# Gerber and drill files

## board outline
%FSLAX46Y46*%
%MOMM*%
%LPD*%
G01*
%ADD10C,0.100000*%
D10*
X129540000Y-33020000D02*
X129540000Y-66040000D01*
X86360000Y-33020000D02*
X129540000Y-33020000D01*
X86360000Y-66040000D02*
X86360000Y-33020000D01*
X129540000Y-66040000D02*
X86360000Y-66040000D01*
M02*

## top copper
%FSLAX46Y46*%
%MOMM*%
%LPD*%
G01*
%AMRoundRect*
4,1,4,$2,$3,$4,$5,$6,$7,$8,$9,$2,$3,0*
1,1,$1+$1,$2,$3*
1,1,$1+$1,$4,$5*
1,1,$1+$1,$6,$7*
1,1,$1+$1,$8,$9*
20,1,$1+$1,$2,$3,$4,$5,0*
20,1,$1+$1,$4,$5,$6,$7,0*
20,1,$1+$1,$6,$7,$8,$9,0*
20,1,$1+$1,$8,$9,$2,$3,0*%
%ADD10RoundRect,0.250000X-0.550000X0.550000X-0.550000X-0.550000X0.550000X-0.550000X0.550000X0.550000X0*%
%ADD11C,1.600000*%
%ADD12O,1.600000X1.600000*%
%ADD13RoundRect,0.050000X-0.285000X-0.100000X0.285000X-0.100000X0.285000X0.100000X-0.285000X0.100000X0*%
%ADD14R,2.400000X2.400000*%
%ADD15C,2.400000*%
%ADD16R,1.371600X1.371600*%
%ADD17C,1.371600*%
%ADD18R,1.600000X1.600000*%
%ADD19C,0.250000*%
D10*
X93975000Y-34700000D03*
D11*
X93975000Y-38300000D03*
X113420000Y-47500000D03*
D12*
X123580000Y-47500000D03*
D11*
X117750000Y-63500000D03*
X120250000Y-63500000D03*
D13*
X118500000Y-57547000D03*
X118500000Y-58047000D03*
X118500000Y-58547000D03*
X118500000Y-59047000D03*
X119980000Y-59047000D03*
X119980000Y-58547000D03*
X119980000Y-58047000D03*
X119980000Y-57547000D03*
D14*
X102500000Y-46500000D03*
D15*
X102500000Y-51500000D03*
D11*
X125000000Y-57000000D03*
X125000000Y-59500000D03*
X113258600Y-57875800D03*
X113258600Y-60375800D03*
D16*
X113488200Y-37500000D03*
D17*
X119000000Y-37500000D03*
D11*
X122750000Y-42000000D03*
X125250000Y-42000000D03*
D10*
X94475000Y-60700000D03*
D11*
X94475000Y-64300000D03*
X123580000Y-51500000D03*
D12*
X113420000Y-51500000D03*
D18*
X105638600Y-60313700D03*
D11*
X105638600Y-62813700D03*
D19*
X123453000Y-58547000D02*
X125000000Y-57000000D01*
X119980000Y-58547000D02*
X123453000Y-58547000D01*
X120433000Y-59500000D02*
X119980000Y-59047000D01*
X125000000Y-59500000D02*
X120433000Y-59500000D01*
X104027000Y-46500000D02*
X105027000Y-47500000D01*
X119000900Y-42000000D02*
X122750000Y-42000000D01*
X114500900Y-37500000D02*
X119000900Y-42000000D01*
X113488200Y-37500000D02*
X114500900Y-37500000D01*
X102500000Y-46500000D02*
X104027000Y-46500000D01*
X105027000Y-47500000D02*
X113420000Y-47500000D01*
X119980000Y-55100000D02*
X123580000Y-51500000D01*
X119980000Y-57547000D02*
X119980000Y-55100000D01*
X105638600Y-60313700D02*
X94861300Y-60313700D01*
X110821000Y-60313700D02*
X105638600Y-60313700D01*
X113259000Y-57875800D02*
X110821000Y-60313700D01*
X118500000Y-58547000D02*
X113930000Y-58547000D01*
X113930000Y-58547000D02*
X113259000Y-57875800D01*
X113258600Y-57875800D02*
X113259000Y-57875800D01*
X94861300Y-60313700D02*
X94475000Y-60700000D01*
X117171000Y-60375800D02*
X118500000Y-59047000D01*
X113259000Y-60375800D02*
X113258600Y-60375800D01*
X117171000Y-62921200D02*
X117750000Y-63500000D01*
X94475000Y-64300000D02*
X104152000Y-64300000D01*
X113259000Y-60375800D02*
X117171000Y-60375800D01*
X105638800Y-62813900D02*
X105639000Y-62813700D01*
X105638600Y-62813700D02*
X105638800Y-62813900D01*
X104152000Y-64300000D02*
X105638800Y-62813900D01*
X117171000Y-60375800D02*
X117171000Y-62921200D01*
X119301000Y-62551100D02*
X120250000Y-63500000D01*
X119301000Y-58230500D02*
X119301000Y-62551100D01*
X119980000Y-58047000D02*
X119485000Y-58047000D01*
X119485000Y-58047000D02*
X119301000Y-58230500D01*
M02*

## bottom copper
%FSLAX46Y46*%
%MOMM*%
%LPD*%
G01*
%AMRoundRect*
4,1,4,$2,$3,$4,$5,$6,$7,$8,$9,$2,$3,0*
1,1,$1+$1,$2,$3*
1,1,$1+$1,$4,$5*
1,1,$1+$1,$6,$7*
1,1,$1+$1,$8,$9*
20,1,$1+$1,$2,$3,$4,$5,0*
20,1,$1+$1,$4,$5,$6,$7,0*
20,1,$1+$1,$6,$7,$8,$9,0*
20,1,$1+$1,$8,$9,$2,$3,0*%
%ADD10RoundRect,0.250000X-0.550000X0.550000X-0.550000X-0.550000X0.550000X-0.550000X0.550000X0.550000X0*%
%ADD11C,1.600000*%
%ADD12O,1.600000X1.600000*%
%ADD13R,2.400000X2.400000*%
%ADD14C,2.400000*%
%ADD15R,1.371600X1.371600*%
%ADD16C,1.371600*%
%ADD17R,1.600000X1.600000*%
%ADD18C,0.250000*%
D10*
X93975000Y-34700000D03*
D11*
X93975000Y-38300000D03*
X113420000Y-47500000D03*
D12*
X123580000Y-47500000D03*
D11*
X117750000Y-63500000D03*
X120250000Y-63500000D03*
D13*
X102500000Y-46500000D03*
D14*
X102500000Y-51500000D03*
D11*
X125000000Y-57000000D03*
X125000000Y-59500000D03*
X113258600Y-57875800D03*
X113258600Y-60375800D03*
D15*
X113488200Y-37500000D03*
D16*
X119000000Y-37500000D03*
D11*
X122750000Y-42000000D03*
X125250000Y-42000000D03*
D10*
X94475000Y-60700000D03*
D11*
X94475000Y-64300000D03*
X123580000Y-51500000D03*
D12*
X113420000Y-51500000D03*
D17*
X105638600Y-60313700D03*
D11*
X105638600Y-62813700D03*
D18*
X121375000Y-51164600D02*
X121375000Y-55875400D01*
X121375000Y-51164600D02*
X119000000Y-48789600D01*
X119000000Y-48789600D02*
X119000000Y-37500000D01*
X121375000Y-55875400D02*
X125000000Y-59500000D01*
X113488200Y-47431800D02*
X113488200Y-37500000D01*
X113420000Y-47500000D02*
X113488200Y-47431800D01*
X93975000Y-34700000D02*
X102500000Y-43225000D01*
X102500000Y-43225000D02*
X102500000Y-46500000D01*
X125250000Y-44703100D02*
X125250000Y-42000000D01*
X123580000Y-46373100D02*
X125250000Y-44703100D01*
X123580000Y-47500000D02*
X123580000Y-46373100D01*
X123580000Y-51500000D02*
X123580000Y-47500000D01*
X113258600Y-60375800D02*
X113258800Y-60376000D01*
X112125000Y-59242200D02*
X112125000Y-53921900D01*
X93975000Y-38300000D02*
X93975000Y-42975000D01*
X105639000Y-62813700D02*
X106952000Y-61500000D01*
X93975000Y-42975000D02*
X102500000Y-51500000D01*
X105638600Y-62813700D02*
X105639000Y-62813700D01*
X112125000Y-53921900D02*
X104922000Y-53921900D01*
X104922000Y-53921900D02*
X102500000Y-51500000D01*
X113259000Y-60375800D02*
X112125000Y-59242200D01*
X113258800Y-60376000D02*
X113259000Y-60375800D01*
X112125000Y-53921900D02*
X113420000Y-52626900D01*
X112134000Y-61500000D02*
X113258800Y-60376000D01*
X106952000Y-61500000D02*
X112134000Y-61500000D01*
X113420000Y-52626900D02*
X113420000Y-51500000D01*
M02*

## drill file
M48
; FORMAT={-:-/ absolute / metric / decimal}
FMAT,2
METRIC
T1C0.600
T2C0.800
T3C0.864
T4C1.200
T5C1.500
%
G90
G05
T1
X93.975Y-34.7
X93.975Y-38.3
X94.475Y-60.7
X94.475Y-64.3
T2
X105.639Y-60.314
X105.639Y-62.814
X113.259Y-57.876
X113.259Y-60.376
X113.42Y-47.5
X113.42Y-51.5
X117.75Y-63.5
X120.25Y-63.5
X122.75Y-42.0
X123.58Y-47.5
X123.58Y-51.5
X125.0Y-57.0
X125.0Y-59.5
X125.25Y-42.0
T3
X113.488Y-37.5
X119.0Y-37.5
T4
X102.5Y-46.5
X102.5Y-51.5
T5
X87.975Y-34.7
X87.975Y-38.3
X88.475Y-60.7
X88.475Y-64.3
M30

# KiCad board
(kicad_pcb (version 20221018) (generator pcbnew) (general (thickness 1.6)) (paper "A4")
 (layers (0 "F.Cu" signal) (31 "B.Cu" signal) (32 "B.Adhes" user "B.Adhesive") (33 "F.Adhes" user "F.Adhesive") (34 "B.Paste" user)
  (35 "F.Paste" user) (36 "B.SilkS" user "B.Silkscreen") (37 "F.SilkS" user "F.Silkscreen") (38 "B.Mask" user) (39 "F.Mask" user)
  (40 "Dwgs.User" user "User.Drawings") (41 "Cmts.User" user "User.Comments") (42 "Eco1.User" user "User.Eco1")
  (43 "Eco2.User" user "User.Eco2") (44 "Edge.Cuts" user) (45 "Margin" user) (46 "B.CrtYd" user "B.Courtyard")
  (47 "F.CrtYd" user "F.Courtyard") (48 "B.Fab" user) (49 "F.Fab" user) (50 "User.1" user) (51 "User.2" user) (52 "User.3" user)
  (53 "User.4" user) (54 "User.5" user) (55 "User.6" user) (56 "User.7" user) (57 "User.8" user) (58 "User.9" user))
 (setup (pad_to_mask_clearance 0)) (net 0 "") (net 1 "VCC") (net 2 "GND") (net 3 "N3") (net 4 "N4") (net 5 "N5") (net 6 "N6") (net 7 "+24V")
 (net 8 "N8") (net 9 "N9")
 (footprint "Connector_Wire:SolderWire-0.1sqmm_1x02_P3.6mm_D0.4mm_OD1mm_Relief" (layer "F.Cu") (at 93.975 34.7 -90)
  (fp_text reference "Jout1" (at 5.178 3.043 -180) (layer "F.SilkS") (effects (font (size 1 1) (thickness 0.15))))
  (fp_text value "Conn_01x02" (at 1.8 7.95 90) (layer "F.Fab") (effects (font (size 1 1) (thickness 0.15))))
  (pad "" np_thru_hole circle (at 0 6 270) (size 1.5 1.5) (drill 1.5) (layers "*.Cu" "*.Mask"))
  (pad "" np_thru_hole circle (at 3.6 6 270) (size 1.5 1.5) (drill 1.5) (layers "*.Cu" "*.Mask"))
  (pad "1" thru_hole roundrect (at 0 0 270) (size 1.6 1.6) (drill 0.6) (layers "*.Cu" "*.Mask") (roundrect_rratio 0.15625) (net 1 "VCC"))
  (pad "2" thru_hole circle (at 3.6 0 270) (size 1.6 1.6) (drill 0.6) (layers "*.Cu" "*.Mask") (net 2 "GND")))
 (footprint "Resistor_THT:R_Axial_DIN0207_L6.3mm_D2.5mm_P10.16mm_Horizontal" (layer "F.Cu") (at 113.42 47.5)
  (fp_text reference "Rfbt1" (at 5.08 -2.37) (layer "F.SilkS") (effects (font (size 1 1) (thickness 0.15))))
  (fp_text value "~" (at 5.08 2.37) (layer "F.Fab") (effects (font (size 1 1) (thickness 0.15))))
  (pad "1" thru_hole circle (at 0 0) (size 1.6 1.6) (drill 0.8) (layers "*.Cu" "*.Mask") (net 1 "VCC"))
  (pad "2" thru_hole oval (at 10.16 0) (size 1.6 1.6) (drill 0.8) (layers "*.Cu" "*.Mask") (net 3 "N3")))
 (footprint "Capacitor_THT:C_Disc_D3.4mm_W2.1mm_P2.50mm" (layer "F.Cu") (at 117.75 63.5)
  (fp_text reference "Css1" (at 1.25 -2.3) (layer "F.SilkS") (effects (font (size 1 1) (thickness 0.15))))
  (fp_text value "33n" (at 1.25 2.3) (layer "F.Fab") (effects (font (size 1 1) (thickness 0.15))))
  (pad "1" thru_hole circle (at 0 0) (size 1.6 1.6) (drill 0.8) (layers "*.Cu" "*.Mask") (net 2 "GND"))
  (pad "2" thru_hole circle (at 2.5 0) (size 1.6 1.6) (drill 0.8) (layers "*.Cu" "*.Mask") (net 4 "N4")))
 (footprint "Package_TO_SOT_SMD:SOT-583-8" (layer "F.Cu") (at 119.24 58.297)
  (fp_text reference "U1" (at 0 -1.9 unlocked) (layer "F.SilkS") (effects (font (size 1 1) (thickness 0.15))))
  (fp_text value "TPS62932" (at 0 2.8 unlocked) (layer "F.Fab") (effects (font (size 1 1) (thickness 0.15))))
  (pad "1" smd roundrect (at -0.74 -0.75) (size 0.67 0.3) (layers "F.Cu" "F.Paste" "F.Mask") (roundrect_rratio 0.1666666667) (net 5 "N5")
   (thermal_bridge_angle 45))
  (pad "2" smd roundrect (at -0.74 -0.25) (size 0.67 0.3) (layers "F.Cu" "F.Paste" "F.Mask") (roundrect_rratio 0.1666666667) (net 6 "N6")
   (thermal_bridge_angle 45))
  (pad "3" smd roundrect (at -0.74 0.25) (size 0.67 0.3) (layers "F.Cu" "F.Paste" "F.Mask") (roundrect_rratio 0.1666666667) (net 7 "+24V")
   (thermal_bridge_angle 45))
  (pad "4" smd roundrect (at -0.74 0.75) (size 0.67 0.3) (layers "F.Cu" "F.Paste" "F.Mask") (roundrect_rratio 0.1666666667) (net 2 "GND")
   (thermal_bridge_angle 45))
  (pad "5" smd roundrect (at 0.74 0.75) (size 0.67 0.3) (layers "F.Cu" "F.Paste" "F.Mask") (roundrect_rratio 0.1666666667) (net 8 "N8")
   (thermal_bridge_angle 45))
  (pad "6" smd roundrect (at 0.74 0.25) (size 0.67 0.3) (layers "F.Cu" "F.Paste" "F.Mask") (roundrect_rratio 0.1666666667) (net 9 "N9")
   (thermal_bridge_angle 45))
  (pad "7" smd roundrect (at 0.74 -0.25) (size 0.67 0.3) (layers "F.Cu" "F.Paste" "F.Mask") (roundrect_rratio 0.1666666667) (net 4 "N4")
   (thermal_bridge_angle 45))
  (pad "8" smd roundrect (at 0.74 -0.75) (size 0.67 0.3) (layers "F.Cu" "F.Paste" "F.Mask") (roundrect_rratio 0.1666666667) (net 3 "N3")
   (thermal_bridge_angle 45)))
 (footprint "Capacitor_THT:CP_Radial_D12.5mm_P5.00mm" (layer "F.Cu") (at 102.5 46.5 -90)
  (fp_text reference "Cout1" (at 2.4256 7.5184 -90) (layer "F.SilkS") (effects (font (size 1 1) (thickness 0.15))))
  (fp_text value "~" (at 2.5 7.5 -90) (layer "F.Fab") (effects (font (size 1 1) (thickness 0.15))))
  (pad "1" thru_hole rect (at 0 0 270) (size 2.4 2.4) (drill 1.2) (layers "*.Cu" "*.Mask") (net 1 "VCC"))
  (pad "2" thru_hole circle (at 5 0 270) (size 2.4 2.4) (drill 1.2) (layers "*.Cu" "*.Mask") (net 2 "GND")))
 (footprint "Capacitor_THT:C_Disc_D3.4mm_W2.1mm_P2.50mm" (layer "F.Cu") (at 125 57 -90)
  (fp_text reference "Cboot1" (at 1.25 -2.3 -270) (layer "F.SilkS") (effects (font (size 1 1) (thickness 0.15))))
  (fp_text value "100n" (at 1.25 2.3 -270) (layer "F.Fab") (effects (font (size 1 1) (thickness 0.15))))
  (pad "1" thru_hole circle (at 0 0 270) (size 1.6 1.6) (drill 0.8) (layers "*.Cu" "*.Mask") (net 9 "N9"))
  (pad "2" thru_hole circle (at 2.5 0 270) (size 1.6 1.6) (drill 0.8) (layers "*.Cu" "*.Mask") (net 8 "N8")))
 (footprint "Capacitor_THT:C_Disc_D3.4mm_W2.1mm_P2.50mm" (layer "F.Cu") (at 113.2586 57.8758 -90)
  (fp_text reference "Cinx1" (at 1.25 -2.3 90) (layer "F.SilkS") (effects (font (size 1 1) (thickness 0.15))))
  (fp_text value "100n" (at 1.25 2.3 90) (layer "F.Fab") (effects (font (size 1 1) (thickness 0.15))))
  (pad "1" thru_hole circle (at 0 0 270) (size 1.6 1.6) (drill 0.8) (layers "*.Cu" "*.Mask") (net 7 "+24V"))
  (pad "2" thru_hole circle (at 2.5 0 270) (size 1.6 1.6) (drill 0.8) (layers "*.Cu" "*.Mask") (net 2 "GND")))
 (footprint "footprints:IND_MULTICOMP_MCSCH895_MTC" (layer "F.Cu") (at 113.4882 37.5)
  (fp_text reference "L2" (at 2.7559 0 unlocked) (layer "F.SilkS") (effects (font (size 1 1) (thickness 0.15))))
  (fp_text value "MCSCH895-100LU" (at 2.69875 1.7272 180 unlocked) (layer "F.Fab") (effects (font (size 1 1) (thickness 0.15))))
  (pad "1" thru_hole rect (at 0 0) (size 1.3716 1.3716) (drill 0.8636) (layers "*.Cu" "*.Mask") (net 1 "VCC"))
  (pad "2" thru_hole circle (at 5.5118 0) (size 1.3716 1.3716) (drill 0.8636) (layers "*.Cu" "*.Mask") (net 8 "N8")))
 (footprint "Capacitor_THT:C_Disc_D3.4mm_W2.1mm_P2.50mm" (layer "F.Cu") (at 122.75 42)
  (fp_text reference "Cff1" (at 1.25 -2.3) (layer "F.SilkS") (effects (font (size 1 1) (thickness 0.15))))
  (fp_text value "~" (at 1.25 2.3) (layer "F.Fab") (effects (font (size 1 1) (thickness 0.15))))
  (pad "1" thru_hole circle (at 0 0) (size 1.6 1.6) (drill 0.8) (layers "*.Cu" "*.Mask") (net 1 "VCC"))
  (pad "2" thru_hole circle (at 2.5 0) (size 1.6 1.6) (drill 0.8) (layers "*.Cu" "*.Mask") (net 3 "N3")))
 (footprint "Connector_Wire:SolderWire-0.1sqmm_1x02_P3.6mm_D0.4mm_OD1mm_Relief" (layer "F.Cu") (at 94.475 60.7 -90)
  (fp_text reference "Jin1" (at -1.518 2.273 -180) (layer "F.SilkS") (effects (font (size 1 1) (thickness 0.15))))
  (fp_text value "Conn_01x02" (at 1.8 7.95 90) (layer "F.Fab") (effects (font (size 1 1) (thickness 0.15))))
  (pad "" np_thru_hole circle (at 0 6 270) (size 1.5 1.5) (drill 1.5) (layers "*.Cu" "*.Mask"))
  (pad "" np_thru_hole circle (at 3.6 6 270) (size 1.5 1.5) (drill 1.5) (layers "*.Cu" "*.Mask"))
  (pad "1" thru_hole roundrect (at 0 0 270) (size 1.6 1.6) (drill 0.6) (layers "*.Cu" "*.Mask") (roundrect_rratio 0.15625) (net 7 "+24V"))
  (pad "2" thru_hole circle (at 3.6 0 270) (size 1.6 1.6) (drill 0.6) (layers "*.Cu" "*.Mask") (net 2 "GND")))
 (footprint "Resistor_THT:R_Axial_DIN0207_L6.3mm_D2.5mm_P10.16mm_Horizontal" (layer "F.Cu") (at 123.58 51.5 180)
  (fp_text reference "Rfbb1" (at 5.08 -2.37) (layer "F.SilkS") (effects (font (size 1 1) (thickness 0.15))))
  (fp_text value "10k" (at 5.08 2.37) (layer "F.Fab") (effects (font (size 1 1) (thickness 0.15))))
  (pad "1" thru_hole circle (at 0 0 180) (size 1.6 1.6) (drill 0.8) (layers "*.Cu" "*.Mask") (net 3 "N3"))
  (pad "2" thru_hole oval (at 10.16 0 180) (size 1.6 1.6) (drill 0.8) (layers "*.Cu" "*.Mask") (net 2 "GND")))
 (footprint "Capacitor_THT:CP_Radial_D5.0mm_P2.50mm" (layer "F.Cu") (at 105.6386 60.3137 -90)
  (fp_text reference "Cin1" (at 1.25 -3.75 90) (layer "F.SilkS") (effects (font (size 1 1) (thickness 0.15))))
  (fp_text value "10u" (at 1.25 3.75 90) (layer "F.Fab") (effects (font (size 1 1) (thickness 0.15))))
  (pad "1" thru_hole rect (at 0 0 270) (size 1.6 1.6) (drill 0.8) (layers "*.Cu" "*.Mask") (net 7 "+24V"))
  (pad "2" thru_hole circle (at 2.5 0 270) (size 1.6 1.6) (drill 0.8) (layers "*.Cu" "*.Mask") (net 2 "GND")))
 (gr_line (start 129.54 33.02) (end 129.54 66.04) (stroke (width 0.1) (type default)) (layer "Edge.Cuts"))
 (gr_line (start 86.36 33.02) (end 129.54 33.02) (stroke (width 0.1) (type default)) (layer "Edge.Cuts"))
 (gr_line (start 86.36 66.04) (end 86.36 33.02) (stroke (width 0.1) (type default)) (layer "Edge.Cuts"))
 (gr_line (start 129.54 66.04) (end 86.36 66.04) (stroke (width 0.1) (type default)) (layer "Edge.Cuts"))
 (segment (start 123.453 58.547) (end 125 57) (width 0.25) (layer "F.Cu") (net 9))
 (segment (start 119.98 58.547) (end 123.453 58.547) (width 0.25) (layer "F.Cu") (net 9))
 (segment (start 120.433 59.5) (end 119.98 59.047) (width 0.25) (layer "F.Cu") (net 8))
 (segment (start 125 59.5) (end 120.433 59.5) (width 0.25) (layer "F.Cu") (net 8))
 (segment (start 121.375 51.1646) (end 121.375 55.8754) (width 0.25) (layer "B.Cu") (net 8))
 (segment (start 121.375 51.1646) (end 119 48.7896) (width 0.25) (layer "B.Cu") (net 8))
 (segment (start 119 48.7896) (end 119 37.5) (width 0.25) (layer "B.Cu") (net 8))
 (segment (start 121.375 55.8754) (end 125 59.5) (width 0.25) (layer "B.Cu") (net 8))
 (segment (start 104.027 46.5) (end 105.027 47.5) (width 0.25) (layer "F.Cu") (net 1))
 (segment (start 119.0009 42) (end 122.75 42) (width 0.25) (layer "F.Cu") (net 1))
 (segment (start 114.5009 37.5) (end 119.0009 42) (width 0.25) (layer "F.Cu") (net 1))
 (segment (start 113.4882 37.5) (end 114.5009 37.5) (width 0.25) (layer "F.Cu") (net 1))
 (segment (start 102.5 46.5) (end 104.027 46.5) (width 0.25) (layer "F.Cu") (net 1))
 (segment (start 105.027 47.5) (end 113.42 47.5) (width 0.25) (layer "F.Cu") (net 1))
 (segment (start 113.4882 47.4318) (end 113.4882 37.5) (width 0.25) (layer "B.Cu") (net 1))
 (segment (start 113.42 47.5) (end 113.4882 47.4318) (width 0.25) (layer "B.Cu") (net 1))
 (segment (start 93.975 34.7) (end 102.5 43.225) (width 0.25) (layer "B.Cu") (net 1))
 (segment (start 102.5 43.225) (end 102.5 46.5) (width 0.25) (layer "B.Cu") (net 1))
 (segment (start 119.98 55.1) (end 123.58 51.5) (width 0.25) (layer "F.Cu") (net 3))
 (segment (start 119.98 57.547) (end 119.98 55.1) (width 0.25) (layer "F.Cu") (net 3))
 (segment (start 125.25 44.7031) (end 125.25 42) (width 0.25) (layer "B.Cu") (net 3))
 (segment (start 123.58 46.3731) (end 125.25 44.7031) (width 0.25) (layer "B.Cu") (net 3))
 (segment (start 123.58 47.5) (end 123.58 46.3731) (width 0.25) (layer "B.Cu") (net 3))
 (segment (start 123.58 51.5) (end 123.58 47.5) (width 0.25) (layer "B.Cu") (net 3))
 (segment (start 105.6386 60.3137) (end 94.8613 60.3137) (width 0.25) (layer "F.Cu") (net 7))
 (segment (start 110.821 60.3137) (end 105.6386 60.3137) (width 0.25) (layer "F.Cu") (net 7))
 (segment (start 113.259 57.8758) (end 110.821 60.3137) (width 0.25) (layer "F.Cu") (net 7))
 (segment (start 118.5 58.547) (end 113.93 58.547) (width 0.25) (layer "F.Cu") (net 7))
 (segment (start 113.93 58.547) (end 113.259 57.8758) (width 0.25) (layer "F.Cu") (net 7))
 (segment (start 113.2586 57.8758) (end 113.259 57.8758) (width 0.25) (layer "F.Cu") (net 7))
 (segment (start 94.8613 60.3137) (end 94.475 60.7) (width 0.25) (layer "F.Cu") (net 7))
 (segment (start 117.171 60.3758) (end 118.5 59.047) (width 0.25) (layer "F.Cu") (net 2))
 (segment (start 113.259 60.3758) (end 113.2586 60.3758) (width 0.25) (layer "F.Cu") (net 2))
 (segment (start 117.171 62.9212) (end 117.75 63.5) (width 0.25) (layer "F.Cu") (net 2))
 (segment (start 94.475 64.3) (end 104.152 64.3) (width 0.25) (layer "F.Cu") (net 2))
 (segment (start 113.259 60.3758) (end 117.171 60.3758) (width 0.25) (layer "F.Cu") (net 2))
 (segment (start 105.6388 62.8139) (end 105.639 62.8137) (width 0.25) (layer "F.Cu") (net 2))
 (segment (start 105.6386 62.8137) (end 105.6388 62.8139) (width 0.25) (layer "F.Cu") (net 2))
 (segment (start 104.152 64.3) (end 105.6388 62.8139) (width 0.25) (layer "F.Cu") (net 2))
 (segment (start 117.171 60.3758) (end 117.171 62.9212) (width 0.25) (layer "F.Cu") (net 2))
 (segment (start 113.2586 60.3758) (end 113.2588 60.376) (width 0.25) (layer "B.Cu") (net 2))
 (segment (start 112.125 59.2422) (end 112.125 53.9219) (width 0.25) (layer "B.Cu") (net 2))
 (segment (start 93.975 38.3) (end 93.975 42.975) (width 0.25) (layer "B.Cu") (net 2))
 (segment (start 105.639 62.8137) (end 106.952 61.5) (width 0.25) (layer "B.Cu") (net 2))
 (segment (start 93.975 42.975) (end 102.5 51.5) (width 0.25) (layer "B.Cu") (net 2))
 (segment (start 105.6386 62.8137) (end 105.639 62.8137) (width 0.25) (layer "B.Cu") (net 2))
 (segment (start 112.125 53.9219) (end 104.922 53.9219) (width 0.25) (layer "B.Cu") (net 2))
 (segment (start 104.922 53.9219) (end 102.5 51.5) (width 0.25) (layer "B.Cu") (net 2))
 (segment (start 113.259 60.3758) (end 112.125 59.2422) (width 0.25) (layer "B.Cu") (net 2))
 (segment (start 113.2588 60.376) (end 113.259 60.3758) (width 0.25) (layer "B.Cu") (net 2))
 (segment (start 112.125 53.9219) (end 113.42 52.6269) (width 0.25) (layer "B.Cu") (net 2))
 (segment (start 112.134 61.5) (end 113.2588 60.376) (width 0.25) (layer "B.Cu") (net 2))
 (segment (start 106.952 61.5) (end 112.134 61.5) (width 0.25) (layer "B.Cu") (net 2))
 (segment (start 113.42 52.6269) (end 113.42 51.5) (width 0.25) (layer "B.Cu") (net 2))
 (segment (start 119.301 62.5511) (end 120.25 63.5) (width 0.25) (layer "F.Cu") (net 4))
 (segment (start 119.301 58.2305) (end 119.301 62.5511) (width 0.25) (layer "F.Cu") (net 4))
 (segment (start 119.98 58.047) (end 119.485 58.047) (width 0.25) (layer "F.Cu") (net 4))
 (segment (start 119.485 58.047) (end 119.301 58.2305) (width 0.25) (layer "F.Cu") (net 4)))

